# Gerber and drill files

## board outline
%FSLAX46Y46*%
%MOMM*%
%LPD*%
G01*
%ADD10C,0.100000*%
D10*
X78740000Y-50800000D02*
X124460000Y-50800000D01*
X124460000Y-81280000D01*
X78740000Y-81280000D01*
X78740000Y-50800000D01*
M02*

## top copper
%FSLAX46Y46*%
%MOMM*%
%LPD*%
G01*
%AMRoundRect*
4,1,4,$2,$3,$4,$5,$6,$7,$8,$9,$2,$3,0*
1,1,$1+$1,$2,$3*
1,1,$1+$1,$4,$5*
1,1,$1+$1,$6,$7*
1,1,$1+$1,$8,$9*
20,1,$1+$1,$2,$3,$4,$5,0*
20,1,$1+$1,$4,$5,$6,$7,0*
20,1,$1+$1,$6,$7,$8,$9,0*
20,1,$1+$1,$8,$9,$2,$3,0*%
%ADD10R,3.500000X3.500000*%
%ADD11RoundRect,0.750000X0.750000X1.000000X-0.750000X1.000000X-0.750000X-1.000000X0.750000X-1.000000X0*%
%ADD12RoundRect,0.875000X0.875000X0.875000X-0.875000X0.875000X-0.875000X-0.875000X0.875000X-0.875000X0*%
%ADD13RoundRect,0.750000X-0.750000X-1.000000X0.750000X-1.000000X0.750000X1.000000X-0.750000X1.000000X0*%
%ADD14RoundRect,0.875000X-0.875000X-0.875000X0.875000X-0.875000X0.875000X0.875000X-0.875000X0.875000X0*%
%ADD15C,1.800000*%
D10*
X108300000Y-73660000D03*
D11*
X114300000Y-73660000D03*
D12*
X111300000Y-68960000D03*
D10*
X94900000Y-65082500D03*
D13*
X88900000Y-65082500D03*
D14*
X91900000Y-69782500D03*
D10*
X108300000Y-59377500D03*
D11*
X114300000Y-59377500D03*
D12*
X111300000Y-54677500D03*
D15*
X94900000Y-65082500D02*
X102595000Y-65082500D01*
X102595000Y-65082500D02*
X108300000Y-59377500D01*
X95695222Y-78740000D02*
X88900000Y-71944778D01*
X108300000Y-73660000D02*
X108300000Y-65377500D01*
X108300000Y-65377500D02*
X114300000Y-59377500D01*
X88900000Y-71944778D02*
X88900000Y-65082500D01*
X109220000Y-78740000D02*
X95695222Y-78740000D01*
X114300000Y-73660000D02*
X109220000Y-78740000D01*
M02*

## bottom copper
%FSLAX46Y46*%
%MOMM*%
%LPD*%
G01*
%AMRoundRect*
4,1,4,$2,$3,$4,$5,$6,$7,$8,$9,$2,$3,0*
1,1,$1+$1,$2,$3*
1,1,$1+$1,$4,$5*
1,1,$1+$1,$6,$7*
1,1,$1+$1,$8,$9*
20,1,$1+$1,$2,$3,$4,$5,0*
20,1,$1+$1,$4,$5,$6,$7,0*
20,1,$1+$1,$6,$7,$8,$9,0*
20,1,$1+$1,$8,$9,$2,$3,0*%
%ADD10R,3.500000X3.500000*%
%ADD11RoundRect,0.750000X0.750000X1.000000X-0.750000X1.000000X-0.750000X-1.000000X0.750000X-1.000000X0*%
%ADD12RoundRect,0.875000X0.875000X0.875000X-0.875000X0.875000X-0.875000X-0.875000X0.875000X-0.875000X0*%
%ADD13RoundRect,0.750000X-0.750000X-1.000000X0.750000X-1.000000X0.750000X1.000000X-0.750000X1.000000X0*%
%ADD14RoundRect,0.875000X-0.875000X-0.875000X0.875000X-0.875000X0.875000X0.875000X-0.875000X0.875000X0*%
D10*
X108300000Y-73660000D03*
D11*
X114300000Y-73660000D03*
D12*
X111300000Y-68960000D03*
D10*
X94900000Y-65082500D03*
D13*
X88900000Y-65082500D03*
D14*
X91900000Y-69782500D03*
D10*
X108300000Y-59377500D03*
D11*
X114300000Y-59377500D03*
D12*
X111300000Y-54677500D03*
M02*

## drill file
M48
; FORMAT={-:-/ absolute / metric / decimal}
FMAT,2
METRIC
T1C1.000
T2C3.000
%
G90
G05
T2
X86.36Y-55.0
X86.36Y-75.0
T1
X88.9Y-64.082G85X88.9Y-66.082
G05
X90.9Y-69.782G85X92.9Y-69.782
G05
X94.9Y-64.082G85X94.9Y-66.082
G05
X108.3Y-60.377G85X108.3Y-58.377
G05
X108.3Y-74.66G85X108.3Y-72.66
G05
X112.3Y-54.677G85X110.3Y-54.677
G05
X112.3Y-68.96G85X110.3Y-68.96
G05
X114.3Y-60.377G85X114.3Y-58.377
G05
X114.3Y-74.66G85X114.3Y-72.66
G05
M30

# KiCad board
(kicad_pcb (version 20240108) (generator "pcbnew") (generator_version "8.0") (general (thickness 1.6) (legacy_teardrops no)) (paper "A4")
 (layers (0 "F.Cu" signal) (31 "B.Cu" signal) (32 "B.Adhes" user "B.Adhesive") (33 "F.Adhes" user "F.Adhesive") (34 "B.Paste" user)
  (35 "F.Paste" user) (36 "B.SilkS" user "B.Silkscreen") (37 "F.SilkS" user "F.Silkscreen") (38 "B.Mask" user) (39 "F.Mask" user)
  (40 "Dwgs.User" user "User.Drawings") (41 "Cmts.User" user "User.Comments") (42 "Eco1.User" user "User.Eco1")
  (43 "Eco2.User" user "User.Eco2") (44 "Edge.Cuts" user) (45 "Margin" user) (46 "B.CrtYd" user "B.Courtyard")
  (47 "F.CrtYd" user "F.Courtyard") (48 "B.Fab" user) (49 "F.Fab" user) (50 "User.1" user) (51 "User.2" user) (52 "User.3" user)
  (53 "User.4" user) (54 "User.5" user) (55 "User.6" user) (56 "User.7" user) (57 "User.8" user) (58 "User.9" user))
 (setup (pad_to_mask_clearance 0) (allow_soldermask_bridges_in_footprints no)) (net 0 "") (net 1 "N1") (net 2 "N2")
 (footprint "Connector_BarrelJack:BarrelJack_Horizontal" (layer "F.Cu") (at 108.3 73.66 180)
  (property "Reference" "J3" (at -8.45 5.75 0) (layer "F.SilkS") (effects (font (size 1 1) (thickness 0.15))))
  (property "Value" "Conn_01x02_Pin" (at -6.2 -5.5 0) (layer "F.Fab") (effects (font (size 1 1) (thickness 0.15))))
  (pad "1" thru_hole rect (at 0 0 180) (size 3.5 3.5) (drill oval 1 3) (layers "*.Cu" "*.Mask") (remove_unused_layers no) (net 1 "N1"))
  (pad "2" thru_hole roundrect (at -6 0 180) (size 3 3.5) (drill oval 1 3) (layers "*.Cu" "*.Mask") (remove_unused_layers no)
   (roundrect_rratio 0.25) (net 1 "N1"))
  (pad "3" thru_hole roundrect (at -3 4.7 180) (size 3.5 3.5) (drill oval 3 1) (layers "*.Cu" "*.Mask") (remove_unused_layers no)
   (roundrect_rratio 0.25) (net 1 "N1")))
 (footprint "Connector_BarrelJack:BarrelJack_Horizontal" (layer "F.Cu") (at 94.9 65.0825)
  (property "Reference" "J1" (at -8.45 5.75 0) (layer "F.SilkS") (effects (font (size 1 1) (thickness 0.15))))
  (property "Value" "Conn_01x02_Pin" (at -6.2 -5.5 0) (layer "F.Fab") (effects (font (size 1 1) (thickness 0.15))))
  (pad "1" thru_hole rect (at 0 0) (size 3.5 3.5) (drill oval 1 3) (layers "*.Cu" "*.Mask") (remove_unused_layers no) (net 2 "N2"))
  (pad "2" thru_hole roundrect (at -6 0) (size 3 3.5) (drill oval 1 3) (layers "*.Cu" "*.Mask") (remove_unused_layers no)
   (roundrect_rratio 0.25) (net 1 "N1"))
  (pad "3" thru_hole roundrect (at -3 4.7) (size 3.5 3.5) (drill oval 3 1) (layers "*.Cu" "*.Mask") (remove_unused_layers no)
   (roundrect_rratio 0.25) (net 1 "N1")))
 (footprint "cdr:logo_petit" (layer "F.Cu") (at 100 72)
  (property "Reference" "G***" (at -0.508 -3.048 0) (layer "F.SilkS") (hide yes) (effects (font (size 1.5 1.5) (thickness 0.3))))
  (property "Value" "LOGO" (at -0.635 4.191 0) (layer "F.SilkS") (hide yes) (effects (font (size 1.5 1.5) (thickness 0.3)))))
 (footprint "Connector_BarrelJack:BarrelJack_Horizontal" (layer "F.Cu") (at 108.3 59.3775 180)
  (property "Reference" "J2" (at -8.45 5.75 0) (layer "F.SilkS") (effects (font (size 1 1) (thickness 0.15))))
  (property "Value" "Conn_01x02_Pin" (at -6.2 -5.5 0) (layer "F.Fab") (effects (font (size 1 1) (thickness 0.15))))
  (pad "1" thru_hole rect (at 0 0 180) (size 3.5 3.5) (drill oval 1 3) (layers "*.Cu" "*.Mask") (remove_unused_layers no) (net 2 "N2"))
  (pad "2" thru_hole roundrect (at -6 0 180) (size 3 3.5) (drill oval 1 3) (layers "*.Cu" "*.Mask") (remove_unused_layers no)
   (roundrect_rratio 0.25) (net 1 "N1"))
  (pad "3" thru_hole roundrect (at -3 4.7 180) (size 3.5 3.5) (drill oval 3 1) (layers "*.Cu" "*.Mask") (remove_unused_layers no)
   (roundrect_rratio 0.25)))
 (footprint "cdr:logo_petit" (layer "F.Cu") (at 100 56)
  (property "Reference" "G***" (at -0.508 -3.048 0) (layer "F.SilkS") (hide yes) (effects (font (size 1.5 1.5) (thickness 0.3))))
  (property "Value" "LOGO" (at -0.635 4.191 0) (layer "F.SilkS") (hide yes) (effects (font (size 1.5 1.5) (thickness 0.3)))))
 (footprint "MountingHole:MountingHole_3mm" (layer "F.Cu") (at 86.36 75)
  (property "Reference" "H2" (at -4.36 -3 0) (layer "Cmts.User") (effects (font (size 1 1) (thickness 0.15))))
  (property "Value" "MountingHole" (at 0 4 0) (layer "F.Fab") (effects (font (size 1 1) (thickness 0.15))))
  (pad "" np_thru_hole circle (at 0 0) (size 3 3) (drill 3) (layers "*.Cu" "*.Mask")))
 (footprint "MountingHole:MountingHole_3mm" (layer "F.Cu") (at 86.36 55)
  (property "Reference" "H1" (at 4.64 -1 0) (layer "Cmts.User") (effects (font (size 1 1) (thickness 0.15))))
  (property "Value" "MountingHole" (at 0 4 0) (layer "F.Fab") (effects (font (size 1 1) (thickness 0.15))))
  (pad "" np_thru_hole circle (at 0 0) (size 3 3) (drill 3) (layers "*.Cu" "*.Mask")))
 (gr_rect (start 78.74 50.8) (end 124.46 81.28) (stroke (width 0.1) (type default)) (fill none) (layer "Edge.Cuts"))
 (segment (start 94.9 65.0825) (end 102.595 65.0825) (width 1.8) (layer "F.Cu") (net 2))
 (segment (start 102.595 65.0825) (end 108.3 59.3775) (width 1.8) (layer "F.Cu") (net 2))
 (segment (start 95.695222 78.74) (end 88.9 71.944778) (width 1.8) (layer "F.Cu") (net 1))
 (segment (start 108.3 73.66) (end 108.3 65.3775) (width 1.8) (layer "F.Cu") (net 1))
 (segment (start 108.3 65.3775) (end 114.3 59.3775) (width 1.8) (layer "F.Cu") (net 1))
 (segment (start 88.9 71.944778) (end 88.9 65.0825) (width 1.8) (layer "F.Cu") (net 1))
 (segment (start 109.22 78.74) (end 95.695222 78.74) (width 1.8) (layer "F.Cu") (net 1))
 (segment (start 114.3 73.66) (end 109.22 78.74) (width 1.8) (layer "F.Cu") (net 1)))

